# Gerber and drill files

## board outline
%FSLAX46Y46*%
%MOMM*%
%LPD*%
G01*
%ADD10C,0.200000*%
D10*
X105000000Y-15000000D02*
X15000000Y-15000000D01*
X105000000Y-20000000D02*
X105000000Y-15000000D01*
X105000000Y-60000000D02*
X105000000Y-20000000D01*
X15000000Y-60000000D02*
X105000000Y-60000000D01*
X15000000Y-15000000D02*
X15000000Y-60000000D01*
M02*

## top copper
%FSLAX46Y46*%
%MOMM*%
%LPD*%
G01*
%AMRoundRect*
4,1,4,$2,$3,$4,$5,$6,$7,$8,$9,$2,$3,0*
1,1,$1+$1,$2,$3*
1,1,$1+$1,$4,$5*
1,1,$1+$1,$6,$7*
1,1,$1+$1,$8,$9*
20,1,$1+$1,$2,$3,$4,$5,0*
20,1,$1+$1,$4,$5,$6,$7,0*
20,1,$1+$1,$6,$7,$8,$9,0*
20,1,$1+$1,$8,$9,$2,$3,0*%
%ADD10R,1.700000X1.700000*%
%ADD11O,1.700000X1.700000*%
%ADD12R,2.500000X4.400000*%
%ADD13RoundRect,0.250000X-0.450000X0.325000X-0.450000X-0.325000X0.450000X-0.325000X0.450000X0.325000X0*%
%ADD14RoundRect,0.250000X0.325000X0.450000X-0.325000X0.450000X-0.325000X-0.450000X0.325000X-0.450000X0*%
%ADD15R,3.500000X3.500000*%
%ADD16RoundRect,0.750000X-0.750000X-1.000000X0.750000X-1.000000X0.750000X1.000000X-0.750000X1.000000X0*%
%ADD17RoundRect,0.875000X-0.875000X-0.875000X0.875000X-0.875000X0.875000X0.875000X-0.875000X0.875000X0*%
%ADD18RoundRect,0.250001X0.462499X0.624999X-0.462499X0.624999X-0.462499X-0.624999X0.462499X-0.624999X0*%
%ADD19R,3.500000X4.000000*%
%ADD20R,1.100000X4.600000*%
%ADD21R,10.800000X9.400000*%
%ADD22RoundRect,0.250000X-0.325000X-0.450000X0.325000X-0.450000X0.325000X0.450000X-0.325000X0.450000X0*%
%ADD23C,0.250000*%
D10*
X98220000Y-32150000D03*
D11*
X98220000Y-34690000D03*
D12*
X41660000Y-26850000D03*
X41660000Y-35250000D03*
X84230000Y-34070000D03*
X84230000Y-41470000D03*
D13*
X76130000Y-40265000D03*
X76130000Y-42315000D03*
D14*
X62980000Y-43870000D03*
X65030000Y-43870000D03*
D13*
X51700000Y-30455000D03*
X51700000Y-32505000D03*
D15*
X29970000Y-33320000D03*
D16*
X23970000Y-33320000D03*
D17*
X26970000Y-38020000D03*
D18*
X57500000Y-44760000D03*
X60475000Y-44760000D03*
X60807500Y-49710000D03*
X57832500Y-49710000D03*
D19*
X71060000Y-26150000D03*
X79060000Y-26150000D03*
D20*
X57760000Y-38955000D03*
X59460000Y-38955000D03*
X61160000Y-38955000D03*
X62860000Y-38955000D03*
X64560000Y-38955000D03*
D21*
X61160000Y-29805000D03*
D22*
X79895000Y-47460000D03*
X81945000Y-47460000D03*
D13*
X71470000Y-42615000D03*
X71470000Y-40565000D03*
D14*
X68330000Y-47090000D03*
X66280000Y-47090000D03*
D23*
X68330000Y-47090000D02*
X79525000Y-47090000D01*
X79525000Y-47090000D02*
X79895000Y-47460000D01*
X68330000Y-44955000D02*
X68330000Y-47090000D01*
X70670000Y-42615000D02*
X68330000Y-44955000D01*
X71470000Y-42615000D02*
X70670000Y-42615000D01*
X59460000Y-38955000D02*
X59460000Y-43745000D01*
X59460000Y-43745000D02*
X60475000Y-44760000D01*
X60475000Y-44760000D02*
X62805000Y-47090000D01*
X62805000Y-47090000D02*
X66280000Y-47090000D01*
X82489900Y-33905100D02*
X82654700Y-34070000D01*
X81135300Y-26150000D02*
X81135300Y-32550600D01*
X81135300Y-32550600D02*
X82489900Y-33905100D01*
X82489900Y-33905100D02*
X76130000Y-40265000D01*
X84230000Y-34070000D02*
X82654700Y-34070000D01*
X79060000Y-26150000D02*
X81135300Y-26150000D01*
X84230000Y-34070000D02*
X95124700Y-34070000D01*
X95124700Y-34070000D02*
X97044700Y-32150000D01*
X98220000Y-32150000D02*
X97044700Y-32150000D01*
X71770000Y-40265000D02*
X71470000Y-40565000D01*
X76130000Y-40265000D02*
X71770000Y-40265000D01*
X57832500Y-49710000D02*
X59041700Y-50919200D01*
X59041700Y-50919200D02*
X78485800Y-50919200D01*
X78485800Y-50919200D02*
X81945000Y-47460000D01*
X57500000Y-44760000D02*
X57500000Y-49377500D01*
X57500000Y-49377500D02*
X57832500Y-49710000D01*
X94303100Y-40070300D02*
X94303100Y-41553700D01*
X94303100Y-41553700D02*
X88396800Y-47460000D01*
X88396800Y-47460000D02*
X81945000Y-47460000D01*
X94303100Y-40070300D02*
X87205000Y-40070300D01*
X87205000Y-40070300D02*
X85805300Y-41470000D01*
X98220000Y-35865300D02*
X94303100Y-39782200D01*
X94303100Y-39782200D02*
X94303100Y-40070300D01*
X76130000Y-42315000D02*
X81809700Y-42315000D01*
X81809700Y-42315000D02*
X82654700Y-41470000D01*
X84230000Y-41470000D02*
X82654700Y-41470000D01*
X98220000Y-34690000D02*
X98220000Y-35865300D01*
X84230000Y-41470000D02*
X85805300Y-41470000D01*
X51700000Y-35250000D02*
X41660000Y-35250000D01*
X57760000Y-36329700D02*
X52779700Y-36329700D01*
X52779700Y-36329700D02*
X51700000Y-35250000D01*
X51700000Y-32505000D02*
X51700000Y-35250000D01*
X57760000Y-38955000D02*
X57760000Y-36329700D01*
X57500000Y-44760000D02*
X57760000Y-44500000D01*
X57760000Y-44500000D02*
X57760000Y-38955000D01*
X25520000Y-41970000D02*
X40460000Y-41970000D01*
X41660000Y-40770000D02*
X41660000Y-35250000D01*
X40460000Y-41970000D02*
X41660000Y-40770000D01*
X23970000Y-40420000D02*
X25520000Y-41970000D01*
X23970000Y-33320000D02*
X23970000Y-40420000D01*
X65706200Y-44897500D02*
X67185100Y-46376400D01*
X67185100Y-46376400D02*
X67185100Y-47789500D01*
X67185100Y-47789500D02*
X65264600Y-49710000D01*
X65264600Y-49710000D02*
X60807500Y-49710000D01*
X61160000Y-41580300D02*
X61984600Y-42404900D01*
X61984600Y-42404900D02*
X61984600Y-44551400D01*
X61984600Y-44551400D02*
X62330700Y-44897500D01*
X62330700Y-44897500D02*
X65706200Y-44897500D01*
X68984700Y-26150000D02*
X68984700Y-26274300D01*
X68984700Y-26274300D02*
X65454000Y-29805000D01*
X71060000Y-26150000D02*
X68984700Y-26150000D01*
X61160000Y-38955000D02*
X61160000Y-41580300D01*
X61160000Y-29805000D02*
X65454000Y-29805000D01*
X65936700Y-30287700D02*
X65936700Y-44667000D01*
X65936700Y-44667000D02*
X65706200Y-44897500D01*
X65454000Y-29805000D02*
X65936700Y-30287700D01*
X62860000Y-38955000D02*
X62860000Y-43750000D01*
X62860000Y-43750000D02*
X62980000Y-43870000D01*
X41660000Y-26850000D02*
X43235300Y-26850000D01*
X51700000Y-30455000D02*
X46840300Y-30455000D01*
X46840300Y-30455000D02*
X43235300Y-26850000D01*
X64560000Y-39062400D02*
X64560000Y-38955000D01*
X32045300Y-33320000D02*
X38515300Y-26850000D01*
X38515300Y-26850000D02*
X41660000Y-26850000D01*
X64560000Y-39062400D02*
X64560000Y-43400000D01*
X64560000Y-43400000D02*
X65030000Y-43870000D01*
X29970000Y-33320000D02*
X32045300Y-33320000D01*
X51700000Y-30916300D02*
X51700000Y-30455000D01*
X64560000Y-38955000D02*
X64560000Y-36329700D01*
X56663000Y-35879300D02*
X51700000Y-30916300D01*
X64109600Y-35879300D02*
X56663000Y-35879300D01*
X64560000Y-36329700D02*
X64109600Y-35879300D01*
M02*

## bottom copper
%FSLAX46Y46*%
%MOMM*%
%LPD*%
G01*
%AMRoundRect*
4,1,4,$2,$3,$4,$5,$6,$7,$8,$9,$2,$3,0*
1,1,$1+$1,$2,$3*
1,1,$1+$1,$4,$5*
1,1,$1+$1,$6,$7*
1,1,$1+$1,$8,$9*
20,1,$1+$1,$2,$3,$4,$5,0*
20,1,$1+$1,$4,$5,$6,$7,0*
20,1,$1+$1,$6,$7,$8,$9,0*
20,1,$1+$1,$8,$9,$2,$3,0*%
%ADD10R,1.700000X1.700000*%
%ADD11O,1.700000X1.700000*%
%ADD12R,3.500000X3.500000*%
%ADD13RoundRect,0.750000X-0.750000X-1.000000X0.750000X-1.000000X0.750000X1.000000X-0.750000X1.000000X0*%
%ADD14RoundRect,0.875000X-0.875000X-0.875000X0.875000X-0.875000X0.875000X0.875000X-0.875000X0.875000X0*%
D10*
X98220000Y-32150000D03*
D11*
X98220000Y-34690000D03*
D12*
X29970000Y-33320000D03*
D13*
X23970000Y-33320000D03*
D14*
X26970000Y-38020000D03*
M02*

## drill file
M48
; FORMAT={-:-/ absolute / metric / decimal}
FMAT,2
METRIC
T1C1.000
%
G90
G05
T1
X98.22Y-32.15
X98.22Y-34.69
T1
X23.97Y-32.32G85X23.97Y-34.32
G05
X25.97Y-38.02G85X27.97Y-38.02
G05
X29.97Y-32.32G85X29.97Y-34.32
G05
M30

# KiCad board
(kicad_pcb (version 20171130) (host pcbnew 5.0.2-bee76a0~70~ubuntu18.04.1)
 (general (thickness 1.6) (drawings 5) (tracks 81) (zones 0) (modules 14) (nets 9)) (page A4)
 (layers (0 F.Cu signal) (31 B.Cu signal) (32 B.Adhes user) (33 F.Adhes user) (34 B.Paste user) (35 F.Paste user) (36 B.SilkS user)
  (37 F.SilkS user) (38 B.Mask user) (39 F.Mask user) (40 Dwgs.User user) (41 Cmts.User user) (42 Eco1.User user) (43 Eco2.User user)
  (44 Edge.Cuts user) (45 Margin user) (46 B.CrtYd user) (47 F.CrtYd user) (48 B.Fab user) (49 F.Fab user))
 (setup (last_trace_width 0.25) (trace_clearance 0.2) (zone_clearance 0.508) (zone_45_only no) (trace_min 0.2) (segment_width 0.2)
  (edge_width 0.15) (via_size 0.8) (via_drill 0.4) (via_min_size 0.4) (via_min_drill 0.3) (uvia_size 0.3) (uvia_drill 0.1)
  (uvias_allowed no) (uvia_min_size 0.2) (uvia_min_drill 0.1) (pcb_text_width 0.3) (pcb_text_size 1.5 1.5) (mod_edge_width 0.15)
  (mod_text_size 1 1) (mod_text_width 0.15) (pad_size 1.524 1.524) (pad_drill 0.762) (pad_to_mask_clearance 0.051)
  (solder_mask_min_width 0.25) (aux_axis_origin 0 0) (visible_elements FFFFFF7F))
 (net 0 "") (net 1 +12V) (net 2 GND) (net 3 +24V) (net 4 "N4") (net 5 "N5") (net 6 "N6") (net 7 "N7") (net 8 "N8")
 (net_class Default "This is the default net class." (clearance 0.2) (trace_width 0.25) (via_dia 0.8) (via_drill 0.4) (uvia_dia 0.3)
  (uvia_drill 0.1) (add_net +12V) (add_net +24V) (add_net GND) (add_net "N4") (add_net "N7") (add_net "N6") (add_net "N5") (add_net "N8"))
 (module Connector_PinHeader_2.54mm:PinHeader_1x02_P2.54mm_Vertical (layer F.Cu) (at 98.22 32.15)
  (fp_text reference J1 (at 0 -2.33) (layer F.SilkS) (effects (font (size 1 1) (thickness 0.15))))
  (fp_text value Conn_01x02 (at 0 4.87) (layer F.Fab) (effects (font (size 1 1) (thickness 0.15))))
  (pad 1 thru_hole rect (at 0 0) (size 1.7 1.7) (drill 1) (layers *.Cu *.Mask) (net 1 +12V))
  (pad 2 thru_hole oval (at 0 2.54) (size 1.7 1.7) (drill 1) (layers *.Cu *.Mask) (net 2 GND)))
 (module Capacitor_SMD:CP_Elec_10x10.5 (layer F.Cu) (at 41.66 31.05 270)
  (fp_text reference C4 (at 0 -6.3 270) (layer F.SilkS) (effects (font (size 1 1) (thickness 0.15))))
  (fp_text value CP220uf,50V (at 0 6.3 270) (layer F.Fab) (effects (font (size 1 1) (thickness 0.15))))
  (pad 1 smd rect (at -4.2 0 270) (size 4.4 2.5) (layers F.Cu F.Paste F.Mask) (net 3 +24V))
  (pad 2 smd rect (at 4.2 0 270) (size 4.4 2.5) (layers F.Cu F.Paste F.Mask) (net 2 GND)))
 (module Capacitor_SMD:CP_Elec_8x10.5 (layer F.Cu) (at 84.23 37.77 270)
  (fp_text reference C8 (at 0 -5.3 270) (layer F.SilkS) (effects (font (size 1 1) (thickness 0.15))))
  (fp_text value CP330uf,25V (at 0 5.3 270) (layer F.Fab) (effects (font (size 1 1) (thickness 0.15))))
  (pad 1 smd rect (at -3.7 0 270) (size 4.4 2.5) (layers F.Cu F.Paste F.Mask) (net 1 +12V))
  (pad 2 smd rect (at 3.7 0 270) (size 4.4 2.5) (layers F.Cu F.Paste F.Mask) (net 2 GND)))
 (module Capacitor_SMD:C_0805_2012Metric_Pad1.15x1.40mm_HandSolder (layer F.Cu) (at 76.13 41.29 270)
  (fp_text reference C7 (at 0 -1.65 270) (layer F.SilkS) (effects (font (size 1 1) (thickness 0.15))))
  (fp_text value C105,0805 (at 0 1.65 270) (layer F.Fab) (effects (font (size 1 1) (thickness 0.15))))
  (pad 1 smd roundrect (at -1.025 0 270) (size 1.15 1.4) (layers F.Cu F.Paste F.Mask) (roundrect_rratio 0.217391) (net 1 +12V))
  (pad 2 smd roundrect (at 1.025 0 270) (size 1.15 1.4) (layers F.Cu F.Paste F.Mask) (roundrect_rratio 0.217391) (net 2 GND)))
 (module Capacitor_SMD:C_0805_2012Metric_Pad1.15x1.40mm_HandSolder (layer F.Cu) (at 64.005 43.87 180)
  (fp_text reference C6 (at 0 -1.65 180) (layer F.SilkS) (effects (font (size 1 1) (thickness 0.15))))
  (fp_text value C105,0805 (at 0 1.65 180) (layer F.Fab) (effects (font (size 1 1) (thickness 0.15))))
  (pad 2 smd roundrect (at 1.025 0 180) (size 1.15 1.4) (layers F.Cu F.Paste F.Mask) (roundrect_rratio 0.217391) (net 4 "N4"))
  (pad 1 smd roundrect (at -1.025 0 180) (size 1.15 1.4) (layers F.Cu F.Paste F.Mask) (roundrect_rratio 0.217391) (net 3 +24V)))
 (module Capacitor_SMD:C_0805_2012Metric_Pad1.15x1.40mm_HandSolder (layer F.Cu) (at 51.7 31.48 270)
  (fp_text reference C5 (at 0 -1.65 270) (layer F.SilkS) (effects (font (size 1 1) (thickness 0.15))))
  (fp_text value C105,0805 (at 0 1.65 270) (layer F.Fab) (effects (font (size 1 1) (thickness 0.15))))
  (pad 1 smd roundrect (at -1.025 0 270) (size 1.15 1.4) (layers F.Cu F.Paste F.Mask) (roundrect_rratio 0.217391) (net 3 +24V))
  (pad 2 smd roundrect (at 1.025 0 270) (size 1.15 1.4) (layers F.Cu F.Paste F.Mask) (roundrect_rratio 0.217391) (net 2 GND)))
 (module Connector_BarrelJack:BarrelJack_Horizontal (layer F.Cu) (at 29.97 33.32)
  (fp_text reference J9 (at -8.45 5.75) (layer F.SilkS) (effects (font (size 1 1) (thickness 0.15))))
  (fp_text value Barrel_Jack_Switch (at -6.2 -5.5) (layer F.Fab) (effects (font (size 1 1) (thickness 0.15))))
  (pad 1 thru_hole rect (at 0 0) (size 3.5 3.5) (drill oval 1 3) (layers *.Cu *.Mask) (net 3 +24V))
  (pad 2 thru_hole roundrect (at -6 0) (size 3 3.5) (drill oval 1 3) (layers *.Cu *.Mask) (roundrect_rratio 0.25) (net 2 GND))
  (pad 3 thru_hole roundrect (at -3 4.7) (size 3.5 3.5) (drill oval 3 1) (layers *.Cu *.Mask) (roundrect_rratio 0.25) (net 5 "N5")))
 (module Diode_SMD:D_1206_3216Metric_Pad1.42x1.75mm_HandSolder (layer F.Cu) (at 58.9875 44.76 180)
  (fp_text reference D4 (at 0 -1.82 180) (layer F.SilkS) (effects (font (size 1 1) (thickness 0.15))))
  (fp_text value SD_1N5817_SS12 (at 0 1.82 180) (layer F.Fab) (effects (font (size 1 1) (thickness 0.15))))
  (pad 2 smd roundrect (at 1.4875 0 180) (size 1.425 1.75) (layers F.Cu F.Paste F.Mask) (roundrect_rratio 0.175439) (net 2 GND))
  (pad 1 smd roundrect (at -1.4875 0 180) (size 1.425 1.75) (layers F.Cu F.Paste F.Mask) (roundrect_rratio 0.175439) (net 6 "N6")))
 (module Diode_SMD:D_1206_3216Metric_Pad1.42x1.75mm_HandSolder (layer F.Cu) (at 59.32 49.71 180)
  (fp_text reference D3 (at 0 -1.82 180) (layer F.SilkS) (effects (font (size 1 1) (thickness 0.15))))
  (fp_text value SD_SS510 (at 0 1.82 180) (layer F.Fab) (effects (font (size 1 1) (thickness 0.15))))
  (pad 1 smd roundrect (at -1.4875 0 180) (size 1.425 1.75) (layers F.Cu F.Paste F.Mask) (roundrect_rratio 0.175439) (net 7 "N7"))
  (pad 2 smd roundrect (at 1.4875 0 180) (size 1.425 1.75) (layers F.Cu F.Paste F.Mask) (roundrect_rratio 0.175439) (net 2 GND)))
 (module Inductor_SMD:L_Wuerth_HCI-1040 (layer F.Cu) (at 75.06 26.15)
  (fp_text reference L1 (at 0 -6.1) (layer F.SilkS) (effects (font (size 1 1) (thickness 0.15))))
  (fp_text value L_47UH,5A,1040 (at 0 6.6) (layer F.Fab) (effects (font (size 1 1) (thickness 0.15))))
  (pad 1 smd rect (at -4 0) (size 3.5 4) (layers F.Cu F.Paste F.Mask) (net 7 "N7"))
  (pad 2 smd rect (at 4 0) (size 3.5 4) (layers F.Cu F.Paste F.Mask) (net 1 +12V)))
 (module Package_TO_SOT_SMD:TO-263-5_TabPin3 (layer F.Cu) (at 61.16 33.18 90)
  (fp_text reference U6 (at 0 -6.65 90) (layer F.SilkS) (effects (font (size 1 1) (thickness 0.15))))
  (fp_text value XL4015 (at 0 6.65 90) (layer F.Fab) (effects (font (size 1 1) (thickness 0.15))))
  (pad 1 smd rect (at -5.775 -3.4 90) (size 4.6 1.1) (layers F.Cu F.Paste F.Mask) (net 2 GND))
  (pad 2 smd rect (at -5.775 -1.7 90) (size 4.6 1.1) (layers F.Cu F.Paste F.Mask) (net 6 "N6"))
  (pad 3 smd rect (at -5.775 0 90) (size 4.6 1.1) (layers F.Cu F.Paste F.Mask) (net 7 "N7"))
  (pad 4 smd rect (at -5.775 1.7 90) (size 4.6 1.1) (layers F.Cu F.Paste F.Mask) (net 4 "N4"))
  (pad 5 smd rect (at -5.775 3.4 90) (size 4.6 1.1) (layers F.Cu F.Paste F.Mask) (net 3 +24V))
  (pad 3 smd rect (at 3.375 0 90) (size 9.4 10.8) (layers F.Cu F.Mask) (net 7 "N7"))
  (pad "" smd rect (at 5.8 2.775 90) (size 4.55 5.25) (layers F.Paste))
  (pad "" smd rect (at 0.95 -2.775 90) (size 4.55 5.25) (layers F.Paste))
  (pad "" smd rect (at 5.8 -2.775 90) (size 4.55 5.25) (layers F.Paste))
  (pad "" smd rect (at 0.95 2.775 90) (size 4.55 5.25) (layers F.Paste)))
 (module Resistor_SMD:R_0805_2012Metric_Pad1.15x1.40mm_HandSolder (layer F.Cu) (at 80.92 47.46)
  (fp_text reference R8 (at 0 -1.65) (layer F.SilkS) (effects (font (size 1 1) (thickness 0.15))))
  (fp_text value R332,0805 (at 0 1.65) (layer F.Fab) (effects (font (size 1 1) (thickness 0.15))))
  (pad 1 smd roundrect (at -1.025 0) (size 1.15 1.4) (layers F.Cu F.Paste F.Mask) (roundrect_rratio 0.217391) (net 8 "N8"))
  (pad 2 smd roundrect (at 1.025 0) (size 1.15 1.4) (layers F.Cu F.Paste F.Mask) (roundrect_rratio 0.217391) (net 2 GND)))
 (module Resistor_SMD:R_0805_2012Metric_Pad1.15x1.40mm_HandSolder (layer F.Cu) (at 71.47 41.59 270)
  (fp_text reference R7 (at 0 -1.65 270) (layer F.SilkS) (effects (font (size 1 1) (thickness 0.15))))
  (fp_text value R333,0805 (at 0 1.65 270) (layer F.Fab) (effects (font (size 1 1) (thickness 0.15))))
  (pad 2 smd roundrect (at 1.025 0 270) (size 1.15 1.4) (layers F.Cu F.Paste F.Mask) (roundrect_rratio 0.217391) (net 8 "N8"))
  (pad 1 smd roundrect (at -1.025 0 270) (size 1.15 1.4) (layers F.Cu F.Paste F.Mask) (roundrect_rratio 0.217391) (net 1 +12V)))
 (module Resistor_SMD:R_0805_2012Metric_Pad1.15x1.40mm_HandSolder (layer F.Cu) (at 67.305 47.09 180)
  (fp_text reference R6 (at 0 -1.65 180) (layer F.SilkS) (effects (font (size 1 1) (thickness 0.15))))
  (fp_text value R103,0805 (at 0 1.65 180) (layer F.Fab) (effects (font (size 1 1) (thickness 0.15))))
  (pad 1 smd roundrect (at -1.025 0 180) (size 1.15 1.4) (layers F.Cu F.Paste F.Mask) (roundrect_rratio 0.217391) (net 8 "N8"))
  (pad 2 smd roundrect (at 1.025 0 180) (size 1.15 1.4) (layers F.Cu F.Paste F.Mask) (roundrect_rratio 0.217391) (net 6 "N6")))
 (gr_line (start 105 15) (end 15 15) (layer Edge.Cuts) (width 0.2))
 (gr_line (start 105 20) (end 105 15) (layer Edge.Cuts) (width 0.2))
 (gr_line (start 105 60) (end 105 20) (layer Edge.Cuts) (width 0.2))
 (gr_line (start 15 60) (end 105 60) (layer Edge.Cuts) (width 0.2))
 (gr_line (start 15 15) (end 15 60) (layer Edge.Cuts) (width 0.2))
 (segment (start 68.33 47.09) (end 79.525 47.09) (width 0.25) (layer F.Cu) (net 8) (status 30))
 (segment (start 79.525 47.09) (end 79.895 47.46) (width 0.25) (layer F.Cu) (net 8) (status 30))
 (segment (start 68.33 44.955) (end 68.33 47.09) (width 0.25) (layer F.Cu) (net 8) (status 20))
 (segment (start 70.67 42.615) (end 68.33 44.955) (width 0.25) (layer F.Cu) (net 8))
 (segment (start 71.47 42.615) (end 70.67 42.615) (width 0.25) (layer F.Cu) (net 8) (status 10))
 (segment (start 59.46 38.955) (end 59.46 43.745) (width 0.25) (layer F.Cu) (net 6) (status 10))
 (segment (start 59.46 43.745) (end 60.475 44.76) (width 0.25) (layer F.Cu) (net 6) (status 20))
 (segment (start 60.475 44.76) (end 62.805 47.09) (width 0.25) (layer F.Cu) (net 6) (status 10))
 (segment (start 62.805 47.09) (end 66.28 47.09) (width 0.25) (layer F.Cu) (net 6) (status 20))
 (segment (start 82.4899 33.9051) (end 82.6547 34.07) (width 0.25) (layer F.Cu) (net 1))
 (segment (start 81.1353 26.15) (end 81.1353 32.5506) (width 0.25) (layer F.Cu) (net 1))
 (segment (start 81.1353 32.5506) (end 82.4899 33.9051) (width 0.25) (layer F.Cu) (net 1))
 (segment (start 82.4899 33.9051) (end 76.13 40.265) (width 0.25) (layer F.Cu) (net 1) (status 20))
 (segment (start 84.23 34.07) (end 82.6547 34.07) (width 0.25) (layer F.Cu) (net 1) (status 10))
 (segment (start 79.06 26.15) (end 81.1353 26.15) (width 0.25) (layer F.Cu) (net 1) (status 10))
 (segment (start 84.23 34.07) (end 95.1247 34.07) (width 0.25) (layer F.Cu) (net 1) (status 10))
 (segment (start 95.1247 34.07) (end 97.0447 32.15) (width 0.25) (layer F.Cu) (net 1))
 (segment (start 98.22 32.15) (end 97.0447 32.15) (width 0.25) (layer F.Cu) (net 1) (status 10))
 (segment (start 71.77 40.265) (end 71.47 40.565) (width 0.25) (layer F.Cu) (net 1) (status 30))
 (segment (start 76.13 40.265) (end 71.77 40.265) (width 0.25) (layer F.Cu) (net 1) (status 30))
 (segment (start 57.8325 49.71) (end 59.0417 50.9192) (width 0.25) (layer F.Cu) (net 2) (status 10))
 (segment (start 59.0417 50.9192) (end 78.4858 50.9192) (width 0.25) (layer F.Cu) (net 2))
 (segment (start 78.4858 50.9192) (end 81.945 47.46) (width 0.25) (layer F.Cu) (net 2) (status 20))
 (segment (start 57.5 44.76) (end 57.5 49.3775) (width 0.25) (layer F.Cu) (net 2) (status 30))
 (segment (start 57.5 49.3775) (end 57.8325 49.71) (width 0.25) (layer F.Cu) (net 2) (status 30))
 (segment (start 94.3031 40.0703) (end 94.3031 41.5537) (width 0.25) (layer F.Cu) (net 2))
 (segment (start 94.3031 41.5537) (end 88.3968 47.46) (width 0.25) (layer F.Cu) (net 2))
 (segment (start 88.3968 47.46) (end 81.945 47.46) (width 0.25) (layer F.Cu) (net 2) (status 20))
 (segment (start 94.3031 40.0703) (end 87.205 40.0703) (width 0.25) (layer F.Cu) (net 2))
 (segment (start 87.205 40.0703) (end 85.8053 41.47) (width 0.25) (layer F.Cu) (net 2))
 (segment (start 98.22 35.8653) (end 94.3031 39.7822) (width 0.25) (layer F.Cu) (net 2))
 (segment (start 94.3031 39.7822) (end 94.3031 40.0703) (width 0.25) (layer F.Cu) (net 2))
 (segment (start 76.13 42.315) (end 81.8097 42.315) (width 0.25) (layer F.Cu) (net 2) (status 10))
 (segment (start 81.8097 42.315) (end 82.6547 41.47) (width 0.25) (layer F.Cu) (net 2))
 (segment (start 84.23 41.47) (end 82.6547 41.47) (width 0.25) (layer F.Cu) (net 2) (status 10))
 (segment (start 98.22 34.69) (end 98.22 35.8653) (width 0.25) (layer F.Cu) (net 2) (status 10))
 (segment (start 84.23 41.47) (end 85.8053 41.47) (width 0.25) (layer F.Cu) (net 2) (status 10))
 (segment (start 51.7 35.25) (end 41.66 35.25) (width 0.25) (layer F.Cu) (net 2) (status 20))
 (segment (start 57.76 36.3297) (end 52.7797 36.3297) (width 0.25) (layer F.Cu) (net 2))
 (segment (start 52.7797 36.3297) (end 51.7 35.25) (width 0.25) (layer F.Cu) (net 2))
 (segment (start 51.7 32.505) (end 51.7 35.25) (width 0.25) (layer F.Cu) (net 2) (status 10))
 (segment (start 57.76 38.955) (end 57.76 36.3297) (width 0.25) (layer F.Cu) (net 2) (status 10))
 (segment (start 57.5 44.76) (end 57.76 44.5) (width 0.25) (layer F.Cu) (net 2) (status 30))
 (segment (start 57.76 44.5) (end 57.76 38.955) (width 0.25) (layer F.Cu) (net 2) (status 30))
 (segment (start 25.52 41.97) (end 40.46 41.97) (width 0.25) (layer F.Cu) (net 2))
 (segment (start 41.66 40.77) (end 41.66 35.25) (width 0.25) (layer F.Cu) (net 2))
 (segment (start 40.46 41.97) (end 41.66 40.77) (width 0.25) (layer F.Cu) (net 2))
 (segment (start 23.97 40.42) (end 25.52 41.97) (width 0.25) (layer F.Cu) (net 2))
 (segment (start 23.97 33.32) (end 23.97 40.42) (width 0.25) (layer F.Cu) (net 2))
 (segment (start 65.7062 44.8975) (end 67.1851 46.3764) (width 0.25) (layer F.Cu) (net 7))
 (segment (start 67.1851 46.3764) (end 67.1851 47.7895) (width 0.25) (layer F.Cu) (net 7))
 (segment (start 67.1851 47.7895) (end 65.2646 49.71) (width 0.25) (layer F.Cu) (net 7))
 (segment (start 65.2646 49.71) (end 60.8075 49.71) (width 0.25) (layer F.Cu) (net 7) (status 20))
 (segment (start 61.16 41.5803) (end 61.9846 42.4049) (width 0.25) (layer F.Cu) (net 7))
 (segment (start 61.9846 42.4049) (end 61.9846 44.5514) (width 0.25) (layer F.Cu) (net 7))
 (segment (start 61.9846 44.5514) (end 62.3307 44.8975) (width 0.25) (layer F.Cu) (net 7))
 (segment (start 62.3307 44.8975) (end 65.7062 44.8975) (width 0.25) (layer F.Cu) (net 7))
 (segment (start 68.9847 26.15) (end 68.9847 26.2743) (width 0.25) (layer F.Cu) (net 7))
 (segment (start 68.9847 26.2743) (end 65.454 29.805) (width 0.25) (layer F.Cu) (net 7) (status 20))
 (segment (start 71.06 26.15) (end 68.9847 26.15) (width 0.25) (layer F.Cu) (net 7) (status 10))
 (segment (start 61.16 38.955) (end 61.16 41.5803) (width 0.25) (layer F.Cu) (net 7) (status 10))
 (segment (start 61.16 29.805) (end 65.454 29.805) (width 0.25) (layer F.Cu) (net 7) (status 30))
 (segment (start 65.9367 30.2877) (end 65.9367 44.667) (width 0.25) (layer F.Cu) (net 7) (status 10))
 (segment (start 65.9367 44.667) (end 65.7062 44.8975) (width 0.25) (layer F.Cu) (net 7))
 (segment (start 65.454 29.805) (end 65.9367 30.2877) (width 0.25) (layer F.Cu) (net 7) (status 30))
 (segment (start 62.86 38.955) (end 62.86 43.75) (width 0.25) (layer F.Cu) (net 4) (status 30))
 (segment (start 62.86 43.75) (end 62.98 43.87) (width 0.25) (layer F.Cu) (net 4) (status 30))
 (segment (start 41.66 26.85) (end 43.2353 26.85) (width 0.25) (layer F.Cu) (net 3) (status 10))
 (segment (start 51.7 30.455) (end 46.8403 30.455) (width 0.25) (layer F.Cu) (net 3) (status 10))
 (segment (start 46.8403 30.455) (end 43.2353 26.85) (width 0.25) (layer F.Cu) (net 3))
 (segment (start 64.56 39.0624) (end 64.56 38.955) (width 0.25) (layer F.Cu) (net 3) (status 30))
 (segment (start 32.0453 33.32) (end 38.5153 26.85) (width 0.25) (layer F.Cu) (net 3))
 (segment (start 38.5153 26.85) (end 41.66 26.85) (width 0.25) (layer F.Cu) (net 3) (status 20))
 (segment (start 64.56 39.0624) (end 64.56 43.4) (width 0.25) (layer F.Cu) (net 3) (status 30))
 (segment (start 64.56 43.4) (end 65.03 43.87) (width 0.25) (layer F.Cu) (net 3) (status 30))
 (segment (start 29.97 33.32) (end 32.0453 33.32) (width 0.25) (layer F.Cu) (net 3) (status 10))
 (segment (start 51.7 30.9163) (end 51.7 30.455) (width 0.25) (layer F.Cu) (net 3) (status 30))
 (segment (start 64.56 38.955) (end 64.56 36.3297) (width 0.25) (layer F.Cu) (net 3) (status 10))
 (segment (start 56.663 35.8793) (end 51.7 30.9163) (width 0.25) (layer F.Cu) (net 3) (status 20))
 (segment (start 64.1096 35.8793) (end 56.663 35.8793) (width 0.25) (layer F.Cu) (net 3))
 (segment (start 64.56 36.3297) (end 64.1096 35.8793) (width 0.25) (layer F.Cu) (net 3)))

